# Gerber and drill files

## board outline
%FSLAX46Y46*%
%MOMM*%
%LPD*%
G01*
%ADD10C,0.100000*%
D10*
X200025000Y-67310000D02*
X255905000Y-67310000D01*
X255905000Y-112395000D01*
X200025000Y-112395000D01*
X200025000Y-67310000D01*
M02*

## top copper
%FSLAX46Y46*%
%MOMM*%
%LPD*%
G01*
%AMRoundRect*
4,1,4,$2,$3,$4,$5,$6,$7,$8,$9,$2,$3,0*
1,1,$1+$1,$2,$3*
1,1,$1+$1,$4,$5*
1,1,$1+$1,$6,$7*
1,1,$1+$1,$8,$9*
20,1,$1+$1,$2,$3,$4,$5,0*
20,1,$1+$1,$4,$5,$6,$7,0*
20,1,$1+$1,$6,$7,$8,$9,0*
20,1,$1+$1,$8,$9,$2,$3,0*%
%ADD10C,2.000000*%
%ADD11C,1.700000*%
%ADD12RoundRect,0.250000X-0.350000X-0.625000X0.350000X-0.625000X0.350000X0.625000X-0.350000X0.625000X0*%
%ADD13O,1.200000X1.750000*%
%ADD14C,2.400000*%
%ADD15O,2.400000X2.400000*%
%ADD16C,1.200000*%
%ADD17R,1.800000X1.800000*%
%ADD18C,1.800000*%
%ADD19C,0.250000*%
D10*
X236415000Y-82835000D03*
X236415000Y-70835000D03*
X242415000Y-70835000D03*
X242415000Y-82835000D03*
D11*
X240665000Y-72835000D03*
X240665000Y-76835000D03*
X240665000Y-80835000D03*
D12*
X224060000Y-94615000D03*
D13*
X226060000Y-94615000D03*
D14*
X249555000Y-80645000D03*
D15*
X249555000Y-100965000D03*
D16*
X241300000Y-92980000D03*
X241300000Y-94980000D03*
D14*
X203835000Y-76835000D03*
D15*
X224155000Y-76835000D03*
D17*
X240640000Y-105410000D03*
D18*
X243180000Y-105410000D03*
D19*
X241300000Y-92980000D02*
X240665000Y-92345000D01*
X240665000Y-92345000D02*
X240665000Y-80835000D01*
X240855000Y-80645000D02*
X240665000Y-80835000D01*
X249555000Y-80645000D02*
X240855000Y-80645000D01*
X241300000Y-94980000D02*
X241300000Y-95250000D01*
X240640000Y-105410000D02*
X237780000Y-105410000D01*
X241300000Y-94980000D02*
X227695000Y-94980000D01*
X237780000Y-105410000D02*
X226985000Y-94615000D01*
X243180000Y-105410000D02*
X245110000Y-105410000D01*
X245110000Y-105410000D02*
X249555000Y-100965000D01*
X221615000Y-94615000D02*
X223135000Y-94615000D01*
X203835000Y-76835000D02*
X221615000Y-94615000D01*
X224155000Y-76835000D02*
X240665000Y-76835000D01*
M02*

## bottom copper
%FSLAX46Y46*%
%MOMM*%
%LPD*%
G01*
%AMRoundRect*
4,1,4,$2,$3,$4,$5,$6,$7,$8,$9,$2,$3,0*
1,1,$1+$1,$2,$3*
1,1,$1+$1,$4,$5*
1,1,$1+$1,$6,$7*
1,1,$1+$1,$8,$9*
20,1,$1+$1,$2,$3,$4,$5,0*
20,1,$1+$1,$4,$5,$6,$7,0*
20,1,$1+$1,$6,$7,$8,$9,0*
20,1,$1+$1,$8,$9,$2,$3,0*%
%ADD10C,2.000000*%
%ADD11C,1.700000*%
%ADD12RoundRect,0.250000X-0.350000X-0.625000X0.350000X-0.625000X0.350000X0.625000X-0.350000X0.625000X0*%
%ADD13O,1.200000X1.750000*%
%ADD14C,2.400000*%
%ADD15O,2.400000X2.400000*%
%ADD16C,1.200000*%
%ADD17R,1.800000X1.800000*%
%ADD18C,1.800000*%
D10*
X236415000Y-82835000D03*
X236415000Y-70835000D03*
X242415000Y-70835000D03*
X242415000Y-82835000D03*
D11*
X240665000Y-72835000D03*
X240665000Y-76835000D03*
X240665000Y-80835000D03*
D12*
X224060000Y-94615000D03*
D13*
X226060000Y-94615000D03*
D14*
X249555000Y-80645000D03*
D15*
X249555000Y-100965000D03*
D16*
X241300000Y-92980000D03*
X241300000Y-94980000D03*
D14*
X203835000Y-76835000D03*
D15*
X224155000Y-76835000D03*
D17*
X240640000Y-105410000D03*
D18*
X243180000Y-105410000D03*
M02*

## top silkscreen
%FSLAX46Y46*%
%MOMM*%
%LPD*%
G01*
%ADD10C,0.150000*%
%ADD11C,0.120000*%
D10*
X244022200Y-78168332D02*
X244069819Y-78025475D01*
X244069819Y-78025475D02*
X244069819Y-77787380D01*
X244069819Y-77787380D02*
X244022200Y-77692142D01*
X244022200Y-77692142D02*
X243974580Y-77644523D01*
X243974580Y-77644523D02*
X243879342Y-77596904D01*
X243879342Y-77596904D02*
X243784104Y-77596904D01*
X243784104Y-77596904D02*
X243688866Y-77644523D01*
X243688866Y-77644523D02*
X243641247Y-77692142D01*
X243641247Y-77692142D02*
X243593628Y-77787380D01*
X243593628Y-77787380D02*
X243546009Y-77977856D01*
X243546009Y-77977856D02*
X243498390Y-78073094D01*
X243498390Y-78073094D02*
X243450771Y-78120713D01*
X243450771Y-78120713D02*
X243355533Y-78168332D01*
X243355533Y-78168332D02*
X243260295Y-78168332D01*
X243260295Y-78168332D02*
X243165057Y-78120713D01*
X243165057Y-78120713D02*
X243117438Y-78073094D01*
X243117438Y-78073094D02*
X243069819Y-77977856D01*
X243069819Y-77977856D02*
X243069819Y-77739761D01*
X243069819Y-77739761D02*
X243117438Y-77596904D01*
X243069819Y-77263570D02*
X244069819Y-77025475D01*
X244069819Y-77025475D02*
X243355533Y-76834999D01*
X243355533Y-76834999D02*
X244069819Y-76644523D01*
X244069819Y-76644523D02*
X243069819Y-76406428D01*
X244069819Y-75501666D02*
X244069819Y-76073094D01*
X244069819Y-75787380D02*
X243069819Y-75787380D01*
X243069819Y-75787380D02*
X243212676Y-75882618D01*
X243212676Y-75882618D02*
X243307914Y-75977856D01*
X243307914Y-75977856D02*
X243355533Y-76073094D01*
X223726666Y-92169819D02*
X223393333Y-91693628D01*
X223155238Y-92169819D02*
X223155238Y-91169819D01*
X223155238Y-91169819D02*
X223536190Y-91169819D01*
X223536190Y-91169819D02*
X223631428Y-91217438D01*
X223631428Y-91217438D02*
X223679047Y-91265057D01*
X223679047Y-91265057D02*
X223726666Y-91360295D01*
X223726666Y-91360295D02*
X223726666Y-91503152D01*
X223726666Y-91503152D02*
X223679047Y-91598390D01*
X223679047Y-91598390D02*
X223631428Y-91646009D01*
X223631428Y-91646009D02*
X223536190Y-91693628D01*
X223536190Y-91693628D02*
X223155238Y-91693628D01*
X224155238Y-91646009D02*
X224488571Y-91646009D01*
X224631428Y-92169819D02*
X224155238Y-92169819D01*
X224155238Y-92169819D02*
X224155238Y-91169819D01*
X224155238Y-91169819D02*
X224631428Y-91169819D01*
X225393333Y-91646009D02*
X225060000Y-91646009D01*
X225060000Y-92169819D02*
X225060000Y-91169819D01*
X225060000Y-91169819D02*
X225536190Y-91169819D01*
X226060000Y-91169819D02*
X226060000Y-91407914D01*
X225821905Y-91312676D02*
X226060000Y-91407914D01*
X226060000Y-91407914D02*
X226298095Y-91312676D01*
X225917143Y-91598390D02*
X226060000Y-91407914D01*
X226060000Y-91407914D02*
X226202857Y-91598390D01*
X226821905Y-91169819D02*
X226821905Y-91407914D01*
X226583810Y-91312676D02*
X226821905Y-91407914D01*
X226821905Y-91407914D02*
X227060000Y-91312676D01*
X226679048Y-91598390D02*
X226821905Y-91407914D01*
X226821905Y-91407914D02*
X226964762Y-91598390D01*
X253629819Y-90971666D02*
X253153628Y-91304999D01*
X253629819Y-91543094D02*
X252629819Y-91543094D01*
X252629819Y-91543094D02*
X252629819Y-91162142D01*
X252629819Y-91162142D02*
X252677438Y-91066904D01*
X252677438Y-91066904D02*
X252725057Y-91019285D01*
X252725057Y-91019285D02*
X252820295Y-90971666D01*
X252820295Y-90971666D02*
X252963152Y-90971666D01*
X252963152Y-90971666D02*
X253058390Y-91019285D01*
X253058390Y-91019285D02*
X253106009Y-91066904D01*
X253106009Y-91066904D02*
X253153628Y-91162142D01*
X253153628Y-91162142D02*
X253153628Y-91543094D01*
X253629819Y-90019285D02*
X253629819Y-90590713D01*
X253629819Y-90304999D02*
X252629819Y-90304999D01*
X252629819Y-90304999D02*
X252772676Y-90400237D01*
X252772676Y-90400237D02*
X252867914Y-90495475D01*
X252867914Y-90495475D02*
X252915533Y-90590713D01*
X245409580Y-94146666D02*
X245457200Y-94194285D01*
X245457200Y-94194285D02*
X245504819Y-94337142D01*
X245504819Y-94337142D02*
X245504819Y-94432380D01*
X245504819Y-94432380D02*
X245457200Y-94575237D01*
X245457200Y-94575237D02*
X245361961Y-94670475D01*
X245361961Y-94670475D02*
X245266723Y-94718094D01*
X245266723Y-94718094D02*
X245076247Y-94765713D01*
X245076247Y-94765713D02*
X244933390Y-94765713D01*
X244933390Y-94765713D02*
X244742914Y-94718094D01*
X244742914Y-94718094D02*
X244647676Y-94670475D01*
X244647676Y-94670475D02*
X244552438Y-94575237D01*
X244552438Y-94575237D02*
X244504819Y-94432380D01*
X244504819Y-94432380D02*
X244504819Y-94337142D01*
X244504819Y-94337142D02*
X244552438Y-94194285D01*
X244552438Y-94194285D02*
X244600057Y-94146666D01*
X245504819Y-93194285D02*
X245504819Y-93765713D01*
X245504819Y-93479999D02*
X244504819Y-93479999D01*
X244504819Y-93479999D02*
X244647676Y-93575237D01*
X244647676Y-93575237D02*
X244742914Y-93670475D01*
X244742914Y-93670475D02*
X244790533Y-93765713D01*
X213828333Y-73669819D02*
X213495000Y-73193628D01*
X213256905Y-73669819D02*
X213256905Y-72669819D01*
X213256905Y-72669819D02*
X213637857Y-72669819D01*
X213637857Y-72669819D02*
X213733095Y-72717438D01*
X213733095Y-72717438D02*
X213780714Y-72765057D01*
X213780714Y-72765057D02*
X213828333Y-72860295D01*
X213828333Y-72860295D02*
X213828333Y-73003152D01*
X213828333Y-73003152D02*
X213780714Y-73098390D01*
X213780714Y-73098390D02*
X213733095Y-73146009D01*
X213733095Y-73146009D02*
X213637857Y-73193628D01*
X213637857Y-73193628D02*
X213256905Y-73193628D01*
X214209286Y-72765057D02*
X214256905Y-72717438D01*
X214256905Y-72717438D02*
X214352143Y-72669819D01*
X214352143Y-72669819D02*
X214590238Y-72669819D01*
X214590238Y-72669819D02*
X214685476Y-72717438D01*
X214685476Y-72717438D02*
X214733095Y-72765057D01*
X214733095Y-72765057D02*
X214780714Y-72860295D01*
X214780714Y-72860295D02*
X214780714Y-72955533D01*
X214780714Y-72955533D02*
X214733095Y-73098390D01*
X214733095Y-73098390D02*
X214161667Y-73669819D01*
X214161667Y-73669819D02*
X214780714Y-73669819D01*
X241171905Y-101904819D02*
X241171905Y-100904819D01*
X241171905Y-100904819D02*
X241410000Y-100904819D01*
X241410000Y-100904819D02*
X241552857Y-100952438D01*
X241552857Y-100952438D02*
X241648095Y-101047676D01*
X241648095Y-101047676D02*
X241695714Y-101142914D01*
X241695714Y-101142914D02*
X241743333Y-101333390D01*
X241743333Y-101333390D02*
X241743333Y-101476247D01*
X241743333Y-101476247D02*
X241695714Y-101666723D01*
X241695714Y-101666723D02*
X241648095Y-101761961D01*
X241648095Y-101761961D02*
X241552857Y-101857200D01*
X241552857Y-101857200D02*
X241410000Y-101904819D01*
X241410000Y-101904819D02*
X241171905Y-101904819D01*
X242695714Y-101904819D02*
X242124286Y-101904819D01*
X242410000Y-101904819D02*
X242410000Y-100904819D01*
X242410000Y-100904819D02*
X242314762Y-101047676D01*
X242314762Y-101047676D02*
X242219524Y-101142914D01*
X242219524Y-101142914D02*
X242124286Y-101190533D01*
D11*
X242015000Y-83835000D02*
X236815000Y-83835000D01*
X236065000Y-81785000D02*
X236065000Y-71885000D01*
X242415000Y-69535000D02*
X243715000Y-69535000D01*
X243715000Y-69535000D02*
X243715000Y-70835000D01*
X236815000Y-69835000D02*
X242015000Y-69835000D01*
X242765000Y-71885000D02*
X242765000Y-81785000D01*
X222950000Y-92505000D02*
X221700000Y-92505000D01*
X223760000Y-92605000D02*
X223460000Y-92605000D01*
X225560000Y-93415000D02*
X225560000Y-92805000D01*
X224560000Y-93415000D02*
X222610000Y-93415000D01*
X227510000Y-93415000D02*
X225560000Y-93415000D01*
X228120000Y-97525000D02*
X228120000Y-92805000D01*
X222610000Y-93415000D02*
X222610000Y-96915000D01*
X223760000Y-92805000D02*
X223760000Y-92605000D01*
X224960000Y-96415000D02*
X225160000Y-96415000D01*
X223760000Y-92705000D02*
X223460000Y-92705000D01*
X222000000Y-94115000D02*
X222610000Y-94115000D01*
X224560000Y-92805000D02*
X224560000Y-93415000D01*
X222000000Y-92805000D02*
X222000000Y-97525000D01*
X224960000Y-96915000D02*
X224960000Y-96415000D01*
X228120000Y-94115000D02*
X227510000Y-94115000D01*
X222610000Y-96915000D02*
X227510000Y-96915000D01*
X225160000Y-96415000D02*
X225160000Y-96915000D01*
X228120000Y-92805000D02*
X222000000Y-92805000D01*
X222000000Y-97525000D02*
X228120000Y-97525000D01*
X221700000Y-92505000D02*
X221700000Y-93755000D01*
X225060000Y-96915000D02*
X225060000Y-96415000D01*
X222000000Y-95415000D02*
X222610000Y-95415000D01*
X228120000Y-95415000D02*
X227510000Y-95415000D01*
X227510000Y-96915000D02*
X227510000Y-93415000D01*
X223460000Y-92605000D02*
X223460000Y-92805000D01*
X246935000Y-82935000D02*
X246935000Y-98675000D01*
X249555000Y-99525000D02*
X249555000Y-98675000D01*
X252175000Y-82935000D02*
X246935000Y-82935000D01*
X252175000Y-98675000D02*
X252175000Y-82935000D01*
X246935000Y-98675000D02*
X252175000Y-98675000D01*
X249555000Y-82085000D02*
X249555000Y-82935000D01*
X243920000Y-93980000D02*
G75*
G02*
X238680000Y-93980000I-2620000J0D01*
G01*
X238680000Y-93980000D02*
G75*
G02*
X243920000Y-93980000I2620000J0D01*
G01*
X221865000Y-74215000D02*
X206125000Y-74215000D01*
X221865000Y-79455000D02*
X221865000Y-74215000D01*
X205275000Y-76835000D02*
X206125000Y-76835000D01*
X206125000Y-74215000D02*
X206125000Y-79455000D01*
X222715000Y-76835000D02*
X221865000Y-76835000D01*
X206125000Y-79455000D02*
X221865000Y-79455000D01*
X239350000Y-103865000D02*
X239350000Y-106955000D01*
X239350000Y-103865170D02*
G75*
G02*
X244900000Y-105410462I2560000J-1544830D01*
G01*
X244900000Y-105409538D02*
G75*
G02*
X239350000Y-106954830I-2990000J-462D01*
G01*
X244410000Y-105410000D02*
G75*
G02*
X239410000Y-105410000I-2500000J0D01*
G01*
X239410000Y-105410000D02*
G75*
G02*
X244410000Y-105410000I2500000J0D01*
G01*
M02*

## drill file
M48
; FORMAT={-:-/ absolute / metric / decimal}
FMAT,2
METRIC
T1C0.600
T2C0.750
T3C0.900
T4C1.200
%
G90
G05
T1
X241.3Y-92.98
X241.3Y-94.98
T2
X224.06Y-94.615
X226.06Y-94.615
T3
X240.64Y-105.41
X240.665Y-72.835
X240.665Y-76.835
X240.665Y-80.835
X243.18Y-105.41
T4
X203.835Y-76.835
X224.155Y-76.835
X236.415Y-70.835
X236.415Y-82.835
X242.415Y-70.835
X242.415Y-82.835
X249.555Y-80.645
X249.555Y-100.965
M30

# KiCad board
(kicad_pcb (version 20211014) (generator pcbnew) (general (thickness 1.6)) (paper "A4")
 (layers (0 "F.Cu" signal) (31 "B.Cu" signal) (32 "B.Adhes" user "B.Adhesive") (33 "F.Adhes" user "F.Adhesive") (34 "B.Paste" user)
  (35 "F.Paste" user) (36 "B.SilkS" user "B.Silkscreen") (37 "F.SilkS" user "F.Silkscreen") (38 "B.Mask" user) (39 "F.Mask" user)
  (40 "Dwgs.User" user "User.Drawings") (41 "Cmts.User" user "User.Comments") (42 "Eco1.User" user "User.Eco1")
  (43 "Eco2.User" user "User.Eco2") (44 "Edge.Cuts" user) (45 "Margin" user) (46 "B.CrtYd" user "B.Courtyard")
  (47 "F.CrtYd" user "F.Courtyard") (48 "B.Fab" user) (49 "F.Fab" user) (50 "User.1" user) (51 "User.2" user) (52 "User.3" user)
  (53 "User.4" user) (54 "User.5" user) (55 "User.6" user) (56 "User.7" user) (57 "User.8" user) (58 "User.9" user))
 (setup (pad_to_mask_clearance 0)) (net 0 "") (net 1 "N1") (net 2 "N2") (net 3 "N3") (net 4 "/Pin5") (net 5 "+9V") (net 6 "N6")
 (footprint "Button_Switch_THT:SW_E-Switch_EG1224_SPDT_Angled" (layer "F.Cu") (at 240.665 72.835 -90)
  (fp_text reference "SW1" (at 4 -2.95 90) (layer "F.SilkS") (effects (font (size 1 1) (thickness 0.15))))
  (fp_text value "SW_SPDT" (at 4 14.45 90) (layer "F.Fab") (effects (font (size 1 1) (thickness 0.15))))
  (fp_line (start 11 -1.35) (end 11 3.85) (layer "F.SilkS") (width 0.12))
  (fp_line (start 8.95 4.6) (end -0.95 4.6) (layer "F.SilkS") (width 0.12))
  (fp_line (start -3.3 -1.75) (end -3.3 -3.05) (layer "F.SilkS") (width 0.12))
  (fp_line (start -3.3 -3.05) (end -2 -3.05) (layer "F.SilkS") (width 0.12))
  (fp_line (start -3 3.85) (end -3 -1.35) (layer "F.SilkS") (width 0.12))
  (fp_line (start -0.95 -2.1) (end 8.95 -2.1) (layer "F.SilkS") (width 0.12))
  (pad "" thru_hole circle (at 10 4.25 270) (size 2 2) (drill 1.2) (layers *.Cu *.Mask))
  (pad "" thru_hole circle (at -2 4.25 270) (size 2 2) (drill 1.2) (layers *.Cu *.Mask))
  (pad "" thru_hole circle (at -2 -1.75 270) (size 2 2) (drill 1.2) (layers *.Cu *.Mask))
  (pad "" thru_hole circle (at 10 -1.75 270) (size 2 2) (drill 1.2) (layers *.Cu *.Mask))
  (pad "1" thru_hole circle (at 0 0 270) (size 1.7 1.7) (drill 0.9) (layers *.Cu *.Mask) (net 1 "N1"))
  (pad "2" thru_hole circle (at 4 0 270) (size 1.7 1.7) (drill 0.9) (layers *.Cu *.Mask) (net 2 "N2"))
  (pad "3" thru_hole circle (at 8 0 270) (size 1.7 1.7) (drill 0.9) (layers *.Cu *.Mask) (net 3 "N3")))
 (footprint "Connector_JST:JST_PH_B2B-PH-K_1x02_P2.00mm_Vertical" (layer "F.Cu") (at 224.06 94.615)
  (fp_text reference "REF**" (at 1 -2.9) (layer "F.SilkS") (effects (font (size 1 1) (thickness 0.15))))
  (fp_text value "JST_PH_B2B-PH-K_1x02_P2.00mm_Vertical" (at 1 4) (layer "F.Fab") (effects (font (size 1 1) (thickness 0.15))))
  (fp_line (start -1.11 -2.11) (end -2.36 -2.11) (layer "F.SilkS") (width 0.12))
  (fp_line (start -0.3 -2.01) (end -0.6 -2.01) (layer "F.SilkS") (width 0.12))
  (fp_line (start 1.5 -1.2) (end 1.5 -1.81) (layer "F.SilkS") (width 0.12))
  (fp_line (start 0.5 -1.2) (end -1.45 -1.2) (layer "F.SilkS") (width 0.12))
  (fp_line (start 3.45 -1.2) (end 1.5 -1.2) (layer "F.SilkS") (width 0.12))
  (fp_line (start 4.06 2.91) (end 4.06 -1.81) (layer "F.SilkS") (width 0.12))
  (fp_line (start -1.45 -1.2) (end -1.45 2.3) (layer "F.SilkS") (width 0.12))
  (fp_line (start -0.3 -1.81) (end -0.3 -2.01) (layer "F.SilkS") (width 0.12))
  (fp_line (start 0.9 1.8) (end 1.1 1.8) (layer "F.SilkS") (width 0.12))
  (fp_line (start -0.3 -1.91) (end -0.6 -1.91) (layer "F.SilkS") (width 0.12))
  (fp_line (start -2.06 -0.5) (end -1.45 -0.5) (layer "F.SilkS") (width 0.12))
  (fp_line (start 0.5 -1.81) (end 0.5 -1.2) (layer "F.SilkS") (width 0.12))
  (fp_line (start -2.06 -1.81) (end -2.06 2.91) (layer "F.SilkS") (width 0.12))
  (fp_line (start 0.9 2.3) (end 0.9 1.8) (layer "F.SilkS") (width 0.12))
  (fp_line (start 4.06 -0.5) (end 3.45 -0.5) (layer "F.SilkS") (width 0.12))
  (fp_line (start -1.45 2.3) (end 3.45 2.3) (layer "F.SilkS") (width 0.12))
  (fp_line (start 1.1 1.8) (end 1.1 2.3) (layer "F.SilkS") (width 0.12))
  (fp_line (start 4.06 -1.81) (end -2.06 -1.81) (layer "F.SilkS") (width 0.12))
  (fp_line (start -2.06 2.91) (end 4.06 2.91) (layer "F.SilkS") (width 0.12))
  (fp_line (start -2.36 -2.11) (end -2.36 -0.86) (layer "F.SilkS") (width 0.12))
  (fp_line (start 1 2.3) (end 1 1.8) (layer "F.SilkS") (width 0.12))
  (fp_line (start -2.06 0.8) (end -1.45 0.8) (layer "F.SilkS") (width 0.12))
  (fp_line (start 4.06 0.8) (end 3.45 0.8) (layer "F.SilkS") (width 0.12))
  (fp_line (start 3.45 2.3) (end 3.45 -1.2) (layer "F.SilkS") (width 0.12))
  (fp_line (start -0.6 -2.01) (end -0.6 -1.81) (layer "F.SilkS") (width 0.12))
  (pad "1" thru_hole roundrect (at 0 0) (size 1.2 1.75) (drill 0.75) (layers *.Cu *.Mask) (roundrect_rratio 0.208333))
  (pad "2" thru_hole oval (at 2 0) (size 1.2 1.75) (drill 0.75) (layers *.Cu *.Mask)))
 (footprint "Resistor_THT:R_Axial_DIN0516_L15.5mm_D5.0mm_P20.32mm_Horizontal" (layer "F.Cu") (at 249.555 80.645 -90)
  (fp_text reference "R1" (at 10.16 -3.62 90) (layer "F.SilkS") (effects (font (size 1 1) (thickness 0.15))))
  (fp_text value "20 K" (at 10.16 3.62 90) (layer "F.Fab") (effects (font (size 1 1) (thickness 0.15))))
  (fp_line (start 2.29 2.62) (end 18.03 2.62) (layer "F.SilkS") (width 0.12))
  (fp_line (start 18.88 0) (end 18.03 0) (layer "F.SilkS") (width 0.12))
  (fp_line (start 2.29 -2.62) (end 2.29 2.62) (layer "F.SilkS") (width 0.12))
  (fp_line (start 18.03 -2.62) (end 2.29 -2.62) (layer "F.SilkS") (width 0.12))
  (fp_line (start 18.03 2.62) (end 18.03 -2.62) (layer "F.SilkS") (width 0.12))
  (fp_line (start 1.44 0) (end 2.29 0) (layer "F.SilkS") (width 0.12))
  (pad "1" thru_hole circle (at 0 0 270) (size 2.4 2.4) (drill 1.2) (layers *.Cu *.Mask) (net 3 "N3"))
  (pad "2" thru_hole oval (at 20.32 0 270) (size 2.4 2.4) (drill 1.2) (layers *.Cu *.Mask) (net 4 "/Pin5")))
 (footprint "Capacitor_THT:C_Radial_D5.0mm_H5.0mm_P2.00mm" (layer "F.Cu") (at 241.3 92.98 -90)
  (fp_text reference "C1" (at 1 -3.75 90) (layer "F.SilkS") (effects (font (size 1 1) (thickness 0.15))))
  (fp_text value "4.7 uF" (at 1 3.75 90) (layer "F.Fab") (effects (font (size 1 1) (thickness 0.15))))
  (fp_circle (center 1 0) (end 3.62 0) (layer "F.SilkS") (width 0.12) (fill none))
  (pad "1" thru_hole circle (at 0 0 270) (size 1.2 1.2) (drill 0.6) (layers *.Cu *.Mask) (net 3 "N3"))
  (pad "2" thru_hole circle (at 2 0 270) (size 1.2 1.2) (drill 0.6) (layers *.Cu *.Mask) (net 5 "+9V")))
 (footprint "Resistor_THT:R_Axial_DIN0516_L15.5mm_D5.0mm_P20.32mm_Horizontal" (layer "F.Cu") (at 203.835 76.835)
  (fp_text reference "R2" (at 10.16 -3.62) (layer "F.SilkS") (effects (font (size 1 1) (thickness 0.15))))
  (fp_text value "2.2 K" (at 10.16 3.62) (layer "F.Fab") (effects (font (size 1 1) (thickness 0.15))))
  (fp_line (start 18.03 -2.62) (end 2.29 -2.62) (layer "F.SilkS") (width 0.12))
  (fp_line (start 18.03 2.62) (end 18.03 -2.62) (layer "F.SilkS") (width 0.12))
  (fp_line (start 1.44 0) (end 2.29 0) (layer "F.SilkS") (width 0.12))
  (fp_line (start 2.29 -2.62) (end 2.29 2.62) (layer "F.SilkS") (width 0.12))
  (fp_line (start 18.88 0) (end 18.03 0) (layer "F.SilkS") (width 0.12))
  (fp_line (start 2.29 2.62) (end 18.03 2.62) (layer "F.SilkS") (width 0.12))
  (pad "1" thru_hole circle (at 0 0) (size 2.4 2.4) (drill 1.2) (layers *.Cu *.Mask) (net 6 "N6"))
  (pad "2" thru_hole oval (at 20.32 0) (size 2.4 2.4) (drill 1.2) (layers *.Cu *.Mask) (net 2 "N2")))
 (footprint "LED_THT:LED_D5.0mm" (layer "F.Cu") (at 240.64 105.41)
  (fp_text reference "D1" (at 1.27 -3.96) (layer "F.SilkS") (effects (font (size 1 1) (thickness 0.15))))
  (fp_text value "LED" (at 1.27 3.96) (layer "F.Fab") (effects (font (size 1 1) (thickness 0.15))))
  (fp_line (start -1.29 -1.545) (end -1.29 1.545) (layer "F.SilkS") (width 0.12))
  (fp_arc (start -1.29 -1.54483) (mid 2.072002 -2.880433) (end 4.26 0.000462) (layer "F.SilkS") (width 0.12))
  (fp_arc (start 4.26 -0.000462) (mid 2.072002 2.880433) (end -1.29 1.54483) (layer "F.SilkS") (width 0.12))
  (fp_circle (center 1.27 0) (end 3.77 0) (layer "F.SilkS") (width 0.12) (fill none))
  (pad "1" thru_hole rect (at 0 0) (size 1.8 1.8) (drill 0.9) (layers *.Cu *.Mask) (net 5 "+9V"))
  (pad "2" thru_hole circle (at 2.54 0) (size 1.8 1.8) (drill 0.9) (layers *.Cu *.Mask) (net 4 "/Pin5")))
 (gr_rect (start 200.025 67.31) (end 255.905 112.395) (layer "Edge.Cuts") (width 0.1) (fill none))
 (segment (start 241.3 92.98) (end 240.665 92.345) (width 0.25) (layer "F.Cu") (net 3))
 (segment (start 240.665 92.345) (end 240.665 80.835) (width 0.25) (layer "F.Cu") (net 3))
 (segment (start 240.855 80.645) (end 240.665 80.835) (width 0.25) (layer "F.Cu") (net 3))
 (segment (start 249.555 80.645) (end 240.855 80.645) (width 0.25) (layer "F.Cu") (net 3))
 (segment (start 241.3 94.98) (end 241.3 95.25) (width 0.25) (layer "F.Cu") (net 5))
 (segment (start 240.64 105.41) (end 237.78 105.41) (width 0.25) (layer "F.Cu") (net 5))
 (segment (start 241.3 94.98) (end 227.695 94.98) (width 0.25) (layer "F.Cu") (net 5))
 (segment (start 237.78 105.41) (end 226.985 94.615) (width 0.25) (layer "F.Cu") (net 5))
 (segment (start 243.18 105.41) (end 245.11 105.41) (width 0.25) (layer "F.Cu") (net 4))
 (segment (start 245.11 105.41) (end 249.555 100.965) (width 0.25) (layer "F.Cu") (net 4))
 (segment (start 221.615 94.615) (end 223.135 94.615) (width 0.25) (layer "F.Cu") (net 6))
 (segment (start 203.835 76.835) (end 221.615 94.615) (width 0.25) (layer "F.Cu") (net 6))
 (segment (start 224.155 76.835) (end 240.665 76.835) (width 0.25) (layer "F.Cu") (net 2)))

